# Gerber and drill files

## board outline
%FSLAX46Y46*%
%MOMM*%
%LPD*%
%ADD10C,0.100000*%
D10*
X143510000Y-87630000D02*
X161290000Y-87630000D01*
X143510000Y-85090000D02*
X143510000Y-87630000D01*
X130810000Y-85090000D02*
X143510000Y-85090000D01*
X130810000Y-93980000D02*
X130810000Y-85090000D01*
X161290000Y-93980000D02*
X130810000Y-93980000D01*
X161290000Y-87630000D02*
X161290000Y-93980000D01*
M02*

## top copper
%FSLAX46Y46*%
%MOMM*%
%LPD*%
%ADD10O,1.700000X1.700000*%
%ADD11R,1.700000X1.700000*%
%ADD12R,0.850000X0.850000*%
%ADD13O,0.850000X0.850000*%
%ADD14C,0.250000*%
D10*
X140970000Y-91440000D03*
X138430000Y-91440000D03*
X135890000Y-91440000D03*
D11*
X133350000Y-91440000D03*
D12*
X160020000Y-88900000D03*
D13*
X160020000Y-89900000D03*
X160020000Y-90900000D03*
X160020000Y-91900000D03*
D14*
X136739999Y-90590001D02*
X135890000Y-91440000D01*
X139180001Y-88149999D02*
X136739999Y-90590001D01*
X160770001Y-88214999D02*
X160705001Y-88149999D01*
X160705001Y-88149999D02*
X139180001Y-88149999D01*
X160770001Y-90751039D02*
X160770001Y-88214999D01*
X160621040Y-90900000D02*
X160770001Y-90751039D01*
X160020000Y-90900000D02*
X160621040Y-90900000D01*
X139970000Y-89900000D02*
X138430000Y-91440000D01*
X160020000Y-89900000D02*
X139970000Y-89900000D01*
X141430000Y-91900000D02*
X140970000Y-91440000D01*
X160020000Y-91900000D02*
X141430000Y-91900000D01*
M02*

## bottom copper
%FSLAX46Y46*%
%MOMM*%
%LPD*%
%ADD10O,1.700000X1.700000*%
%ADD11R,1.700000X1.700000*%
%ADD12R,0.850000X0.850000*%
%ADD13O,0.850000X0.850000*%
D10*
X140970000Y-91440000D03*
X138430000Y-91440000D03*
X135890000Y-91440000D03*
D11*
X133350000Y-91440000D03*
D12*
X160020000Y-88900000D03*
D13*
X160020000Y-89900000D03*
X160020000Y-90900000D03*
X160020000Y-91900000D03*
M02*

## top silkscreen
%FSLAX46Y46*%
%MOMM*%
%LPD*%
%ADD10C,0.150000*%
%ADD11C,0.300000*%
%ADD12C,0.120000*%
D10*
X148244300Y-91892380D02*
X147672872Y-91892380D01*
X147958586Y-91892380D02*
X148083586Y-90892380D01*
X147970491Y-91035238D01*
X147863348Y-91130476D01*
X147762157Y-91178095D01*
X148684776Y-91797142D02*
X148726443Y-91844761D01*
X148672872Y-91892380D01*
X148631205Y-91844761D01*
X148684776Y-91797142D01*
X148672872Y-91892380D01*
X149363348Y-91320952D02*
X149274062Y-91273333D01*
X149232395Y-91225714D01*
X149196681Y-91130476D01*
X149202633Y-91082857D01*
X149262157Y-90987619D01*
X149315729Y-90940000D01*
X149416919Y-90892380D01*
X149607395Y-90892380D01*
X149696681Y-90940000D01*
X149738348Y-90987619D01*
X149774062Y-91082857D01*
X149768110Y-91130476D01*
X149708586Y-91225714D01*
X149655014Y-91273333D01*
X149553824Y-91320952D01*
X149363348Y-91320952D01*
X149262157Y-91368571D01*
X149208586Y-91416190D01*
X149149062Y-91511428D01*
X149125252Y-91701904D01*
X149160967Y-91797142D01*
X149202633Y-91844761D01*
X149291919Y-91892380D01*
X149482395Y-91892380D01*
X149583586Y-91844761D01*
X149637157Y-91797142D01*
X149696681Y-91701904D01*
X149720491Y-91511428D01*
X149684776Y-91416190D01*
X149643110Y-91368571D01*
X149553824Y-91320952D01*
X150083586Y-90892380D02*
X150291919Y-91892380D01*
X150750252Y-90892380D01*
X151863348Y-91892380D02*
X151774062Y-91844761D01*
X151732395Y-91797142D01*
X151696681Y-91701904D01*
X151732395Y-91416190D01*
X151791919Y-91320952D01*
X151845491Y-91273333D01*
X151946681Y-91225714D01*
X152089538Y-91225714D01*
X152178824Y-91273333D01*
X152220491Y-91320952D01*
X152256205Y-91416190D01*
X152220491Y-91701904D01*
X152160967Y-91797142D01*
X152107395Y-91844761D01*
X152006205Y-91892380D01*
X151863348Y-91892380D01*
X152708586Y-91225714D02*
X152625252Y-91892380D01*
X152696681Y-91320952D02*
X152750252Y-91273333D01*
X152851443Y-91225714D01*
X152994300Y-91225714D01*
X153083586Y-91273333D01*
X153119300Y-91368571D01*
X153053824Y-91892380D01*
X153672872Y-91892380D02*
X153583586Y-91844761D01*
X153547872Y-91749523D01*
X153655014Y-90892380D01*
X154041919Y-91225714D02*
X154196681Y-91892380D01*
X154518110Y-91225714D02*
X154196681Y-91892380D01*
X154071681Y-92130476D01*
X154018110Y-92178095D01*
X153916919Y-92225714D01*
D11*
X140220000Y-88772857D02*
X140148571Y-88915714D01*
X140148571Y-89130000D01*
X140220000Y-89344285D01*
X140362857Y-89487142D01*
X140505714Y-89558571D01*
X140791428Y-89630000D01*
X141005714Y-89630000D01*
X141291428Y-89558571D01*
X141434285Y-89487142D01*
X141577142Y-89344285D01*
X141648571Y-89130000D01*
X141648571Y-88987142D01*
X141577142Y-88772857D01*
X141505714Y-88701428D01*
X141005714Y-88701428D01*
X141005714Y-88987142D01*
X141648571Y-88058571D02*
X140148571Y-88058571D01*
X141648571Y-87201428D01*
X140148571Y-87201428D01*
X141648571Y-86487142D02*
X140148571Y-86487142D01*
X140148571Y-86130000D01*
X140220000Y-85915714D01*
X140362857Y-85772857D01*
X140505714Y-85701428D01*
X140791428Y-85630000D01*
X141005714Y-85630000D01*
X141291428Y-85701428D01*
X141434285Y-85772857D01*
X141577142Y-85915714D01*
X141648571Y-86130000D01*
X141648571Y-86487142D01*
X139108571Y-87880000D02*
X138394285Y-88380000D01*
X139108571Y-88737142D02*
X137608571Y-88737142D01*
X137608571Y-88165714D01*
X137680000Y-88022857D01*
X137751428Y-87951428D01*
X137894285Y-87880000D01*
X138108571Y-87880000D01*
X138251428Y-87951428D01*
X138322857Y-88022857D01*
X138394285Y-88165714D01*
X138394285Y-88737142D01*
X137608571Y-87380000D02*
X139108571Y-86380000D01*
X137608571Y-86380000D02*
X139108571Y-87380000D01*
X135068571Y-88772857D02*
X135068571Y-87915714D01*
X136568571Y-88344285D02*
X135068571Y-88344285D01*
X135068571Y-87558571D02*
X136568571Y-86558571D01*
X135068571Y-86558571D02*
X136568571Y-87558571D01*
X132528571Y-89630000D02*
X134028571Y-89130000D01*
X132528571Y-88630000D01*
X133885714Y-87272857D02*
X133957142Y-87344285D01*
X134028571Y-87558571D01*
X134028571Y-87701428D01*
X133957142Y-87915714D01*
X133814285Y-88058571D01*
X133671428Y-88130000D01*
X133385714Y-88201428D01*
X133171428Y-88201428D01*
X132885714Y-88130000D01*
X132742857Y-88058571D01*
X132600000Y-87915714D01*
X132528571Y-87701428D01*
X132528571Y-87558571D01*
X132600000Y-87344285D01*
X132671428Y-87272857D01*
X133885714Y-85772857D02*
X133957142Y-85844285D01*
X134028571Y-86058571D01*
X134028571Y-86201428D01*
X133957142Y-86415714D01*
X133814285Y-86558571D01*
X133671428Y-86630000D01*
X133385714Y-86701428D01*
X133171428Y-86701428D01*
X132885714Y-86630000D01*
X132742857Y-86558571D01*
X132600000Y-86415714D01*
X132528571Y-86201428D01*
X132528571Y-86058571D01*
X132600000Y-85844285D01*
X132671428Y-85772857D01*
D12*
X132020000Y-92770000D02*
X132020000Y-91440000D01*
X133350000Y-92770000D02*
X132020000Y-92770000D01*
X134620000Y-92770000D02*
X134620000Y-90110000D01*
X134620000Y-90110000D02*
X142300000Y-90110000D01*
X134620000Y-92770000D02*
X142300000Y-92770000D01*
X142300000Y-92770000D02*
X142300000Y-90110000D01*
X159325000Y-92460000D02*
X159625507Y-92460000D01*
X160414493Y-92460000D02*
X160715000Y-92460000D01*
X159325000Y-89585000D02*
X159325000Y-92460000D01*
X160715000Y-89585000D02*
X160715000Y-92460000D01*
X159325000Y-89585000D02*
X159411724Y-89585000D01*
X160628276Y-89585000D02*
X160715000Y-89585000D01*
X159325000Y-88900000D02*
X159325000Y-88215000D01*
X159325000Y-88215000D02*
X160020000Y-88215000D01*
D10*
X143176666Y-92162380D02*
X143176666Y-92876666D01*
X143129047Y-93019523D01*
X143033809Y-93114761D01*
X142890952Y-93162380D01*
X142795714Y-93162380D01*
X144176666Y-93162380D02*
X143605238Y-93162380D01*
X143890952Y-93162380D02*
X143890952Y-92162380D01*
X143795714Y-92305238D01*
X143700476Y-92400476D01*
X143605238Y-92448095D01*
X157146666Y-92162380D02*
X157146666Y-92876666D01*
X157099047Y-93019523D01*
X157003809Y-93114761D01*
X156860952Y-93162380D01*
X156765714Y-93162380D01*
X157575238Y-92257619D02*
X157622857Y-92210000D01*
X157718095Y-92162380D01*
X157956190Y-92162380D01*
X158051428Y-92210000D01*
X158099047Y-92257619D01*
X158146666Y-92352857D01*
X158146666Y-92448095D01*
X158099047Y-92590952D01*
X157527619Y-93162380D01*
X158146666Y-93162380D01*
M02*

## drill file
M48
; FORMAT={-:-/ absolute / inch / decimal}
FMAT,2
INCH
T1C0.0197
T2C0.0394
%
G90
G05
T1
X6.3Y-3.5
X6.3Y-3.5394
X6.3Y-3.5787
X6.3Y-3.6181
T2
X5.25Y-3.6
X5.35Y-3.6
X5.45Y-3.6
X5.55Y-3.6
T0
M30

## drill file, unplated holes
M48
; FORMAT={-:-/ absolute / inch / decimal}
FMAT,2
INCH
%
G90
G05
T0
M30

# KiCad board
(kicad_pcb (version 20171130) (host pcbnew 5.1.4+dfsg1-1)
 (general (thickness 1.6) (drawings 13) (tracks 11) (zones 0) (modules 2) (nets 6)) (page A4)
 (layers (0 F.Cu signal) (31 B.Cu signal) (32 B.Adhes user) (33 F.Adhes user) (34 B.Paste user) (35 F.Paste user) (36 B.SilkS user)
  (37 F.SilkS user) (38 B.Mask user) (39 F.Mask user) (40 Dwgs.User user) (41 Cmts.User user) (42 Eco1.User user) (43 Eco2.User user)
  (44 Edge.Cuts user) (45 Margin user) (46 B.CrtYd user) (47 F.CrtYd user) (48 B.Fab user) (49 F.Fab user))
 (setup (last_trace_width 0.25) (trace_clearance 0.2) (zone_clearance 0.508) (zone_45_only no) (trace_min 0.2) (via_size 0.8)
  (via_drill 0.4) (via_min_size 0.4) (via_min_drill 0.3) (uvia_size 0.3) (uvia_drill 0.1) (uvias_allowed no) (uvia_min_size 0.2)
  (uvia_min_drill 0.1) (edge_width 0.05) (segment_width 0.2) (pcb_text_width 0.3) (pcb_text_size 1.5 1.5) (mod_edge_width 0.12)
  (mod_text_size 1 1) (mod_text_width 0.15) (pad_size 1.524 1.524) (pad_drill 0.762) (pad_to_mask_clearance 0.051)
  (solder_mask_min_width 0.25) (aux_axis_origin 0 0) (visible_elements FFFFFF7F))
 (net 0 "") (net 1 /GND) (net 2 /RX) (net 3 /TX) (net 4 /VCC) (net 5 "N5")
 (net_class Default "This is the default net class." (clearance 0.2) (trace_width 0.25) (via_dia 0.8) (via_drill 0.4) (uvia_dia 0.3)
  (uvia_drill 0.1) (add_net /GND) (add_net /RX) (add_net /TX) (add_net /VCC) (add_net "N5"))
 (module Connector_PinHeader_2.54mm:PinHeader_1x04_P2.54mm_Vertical (layer F.Cu) (at 133.35 91.44 90)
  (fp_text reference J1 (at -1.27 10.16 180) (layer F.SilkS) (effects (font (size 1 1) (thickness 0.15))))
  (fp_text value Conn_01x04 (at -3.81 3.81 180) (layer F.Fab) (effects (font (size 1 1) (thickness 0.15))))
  (fp_line (start -1.33 -1.33) (end 0 -1.33) (layer F.SilkS) (width 0.12))
  (fp_line (start -1.33 0) (end -1.33 -1.33) (layer F.SilkS) (width 0.12))
  (fp_line (start -1.33 1.27) (end 1.33 1.27) (layer F.SilkS) (width 0.12))
  (fp_line (start 1.33 1.27) (end 1.33 8.95) (layer F.SilkS) (width 0.12))
  (fp_line (start -1.33 1.27) (end -1.33 8.95) (layer F.SilkS) (width 0.12))
  (fp_line (start -1.33 8.95) (end 1.33 8.95) (layer F.SilkS) (width 0.12))
  (pad 4 thru_hole oval (at 0 7.62 90) (size 1.7 1.7) (drill 1) (layers *.Cu *.Mask) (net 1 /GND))
  (pad 3 thru_hole oval (at 0 5.08 90) (size 1.7 1.7) (drill 1) (layers *.Cu *.Mask) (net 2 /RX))
  (pad 2 thru_hole oval (at 0 2.54 90) (size 1.7 1.7) (drill 1) (layers *.Cu *.Mask) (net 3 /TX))
  (pad 1 thru_hole rect (at 0 0 90) (size 1.7 1.7) (drill 1) (layers *.Cu *.Mask) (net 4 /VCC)))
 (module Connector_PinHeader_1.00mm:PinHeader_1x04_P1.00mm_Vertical (layer F.Cu) (at 160.02 88.9)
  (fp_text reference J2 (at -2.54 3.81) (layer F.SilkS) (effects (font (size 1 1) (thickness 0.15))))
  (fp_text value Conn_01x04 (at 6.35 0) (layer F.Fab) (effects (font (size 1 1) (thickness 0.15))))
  (fp_line (start -0.695 3.56) (end -0.394493 3.56) (layer F.SilkS) (width 0.12))
  (fp_line (start 0.394493 3.56) (end 0.695 3.56) (layer F.SilkS) (width 0.12))
  (fp_line (start -0.695 0.685) (end -0.695 3.56) (layer F.SilkS) (width 0.12))
  (fp_line (start 0.695 0.685) (end 0.695 3.56) (layer F.SilkS) (width 0.12))
  (fp_line (start -0.695 0.685) (end -0.608276 0.685) (layer F.SilkS) (width 0.12))
  (fp_line (start 0.608276 0.685) (end 0.695 0.685) (layer F.SilkS) (width 0.12))
  (fp_line (start -0.695 0) (end -0.695 -0.685) (layer F.SilkS) (width 0.12))
  (fp_line (start -0.695 -0.685) (end 0 -0.685) (layer F.SilkS) (width 0.12))
  (pad 1 thru_hole rect (at 0 0) (size 0.85 0.85) (drill 0.5) (layers *.Cu *.Mask) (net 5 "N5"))
  (pad 2 thru_hole oval (at 0 1) (size 0.85 0.85) (drill 0.5) (layers *.Cu *.Mask) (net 2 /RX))
  (pad 3 thru_hole oval (at 0 2) (size 0.85 0.85) (drill 0.5) (layers *.Cu *.Mask) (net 3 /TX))
  (pad 4 thru_hole oval (at 0 3) (size 0.85 0.85) (drill 0.5) (layers *.Cu *.Mask) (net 1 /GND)))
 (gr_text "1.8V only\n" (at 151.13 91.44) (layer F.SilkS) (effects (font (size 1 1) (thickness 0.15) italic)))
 (gr_line (start 143.51 87.63) (end 161.29 87.63) (layer Edge.Cuts) (width 0.1))
 (gr_line (start 143.51 85.09) (end 143.51 87.63) (layer Edge.Cuts) (width 0.1))
 (gr_line (start 130.81 85.09) (end 143.51 85.09) (layer Edge.Cuts) (width 0.1))
 (gr_line (start 130.81 93.98) (end 130.81 85.09) (layer Edge.Cuts) (width 0.1))
 (gr_line (start 161.29 93.98) (end 130.81 93.98) (layer Edge.Cuts) (width 0.1))
 (gr_line (start 161.29 87.63) (end 161.29 93.98) (layer Edge.Cuts) (width 0.1))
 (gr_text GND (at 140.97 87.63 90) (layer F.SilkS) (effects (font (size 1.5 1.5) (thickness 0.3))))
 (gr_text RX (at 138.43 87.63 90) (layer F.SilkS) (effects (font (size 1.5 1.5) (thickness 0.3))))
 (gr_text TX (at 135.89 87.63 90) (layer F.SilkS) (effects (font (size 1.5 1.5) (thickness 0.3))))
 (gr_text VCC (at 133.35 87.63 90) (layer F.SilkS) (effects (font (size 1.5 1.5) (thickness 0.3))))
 (segment (start 136.739999 90.590001) (end 135.89 91.44) (width 0.25) (layer F.Cu) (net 3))
 (segment (start 139.180001 88.149999) (end 136.739999 90.590001) (width 0.25) (layer F.Cu) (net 3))
 (segment (start 160.770001 88.214999) (end 160.705001 88.149999) (width 0.25) (layer F.Cu) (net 3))
 (segment (start 160.705001 88.149999) (end 139.180001 88.149999) (width 0.25) (layer F.Cu) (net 3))
 (segment (start 160.770001 90.751039) (end 160.770001 88.214999) (width 0.25) (layer F.Cu) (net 3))
 (segment (start 160.62104 90.9) (end 160.770001 90.751039) (width 0.25) (layer F.Cu) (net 3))
 (segment (start 160.02 90.9) (end 160.62104 90.9) (width 0.25) (layer F.Cu) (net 3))
 (segment (start 139.97 89.9) (end 138.43 91.44) (width 0.25) (layer F.Cu) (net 2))
 (segment (start 160.02 89.9) (end 139.97 89.9) (width 0.25) (layer F.Cu) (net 2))
 (segment (start 141.43 91.9) (end 140.97 91.44) (width 0.25) (layer F.Cu) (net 1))
 (segment (start 160.02 91.9) (end 141.43 91.9) (width 0.25) (layer F.Cu) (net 1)))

